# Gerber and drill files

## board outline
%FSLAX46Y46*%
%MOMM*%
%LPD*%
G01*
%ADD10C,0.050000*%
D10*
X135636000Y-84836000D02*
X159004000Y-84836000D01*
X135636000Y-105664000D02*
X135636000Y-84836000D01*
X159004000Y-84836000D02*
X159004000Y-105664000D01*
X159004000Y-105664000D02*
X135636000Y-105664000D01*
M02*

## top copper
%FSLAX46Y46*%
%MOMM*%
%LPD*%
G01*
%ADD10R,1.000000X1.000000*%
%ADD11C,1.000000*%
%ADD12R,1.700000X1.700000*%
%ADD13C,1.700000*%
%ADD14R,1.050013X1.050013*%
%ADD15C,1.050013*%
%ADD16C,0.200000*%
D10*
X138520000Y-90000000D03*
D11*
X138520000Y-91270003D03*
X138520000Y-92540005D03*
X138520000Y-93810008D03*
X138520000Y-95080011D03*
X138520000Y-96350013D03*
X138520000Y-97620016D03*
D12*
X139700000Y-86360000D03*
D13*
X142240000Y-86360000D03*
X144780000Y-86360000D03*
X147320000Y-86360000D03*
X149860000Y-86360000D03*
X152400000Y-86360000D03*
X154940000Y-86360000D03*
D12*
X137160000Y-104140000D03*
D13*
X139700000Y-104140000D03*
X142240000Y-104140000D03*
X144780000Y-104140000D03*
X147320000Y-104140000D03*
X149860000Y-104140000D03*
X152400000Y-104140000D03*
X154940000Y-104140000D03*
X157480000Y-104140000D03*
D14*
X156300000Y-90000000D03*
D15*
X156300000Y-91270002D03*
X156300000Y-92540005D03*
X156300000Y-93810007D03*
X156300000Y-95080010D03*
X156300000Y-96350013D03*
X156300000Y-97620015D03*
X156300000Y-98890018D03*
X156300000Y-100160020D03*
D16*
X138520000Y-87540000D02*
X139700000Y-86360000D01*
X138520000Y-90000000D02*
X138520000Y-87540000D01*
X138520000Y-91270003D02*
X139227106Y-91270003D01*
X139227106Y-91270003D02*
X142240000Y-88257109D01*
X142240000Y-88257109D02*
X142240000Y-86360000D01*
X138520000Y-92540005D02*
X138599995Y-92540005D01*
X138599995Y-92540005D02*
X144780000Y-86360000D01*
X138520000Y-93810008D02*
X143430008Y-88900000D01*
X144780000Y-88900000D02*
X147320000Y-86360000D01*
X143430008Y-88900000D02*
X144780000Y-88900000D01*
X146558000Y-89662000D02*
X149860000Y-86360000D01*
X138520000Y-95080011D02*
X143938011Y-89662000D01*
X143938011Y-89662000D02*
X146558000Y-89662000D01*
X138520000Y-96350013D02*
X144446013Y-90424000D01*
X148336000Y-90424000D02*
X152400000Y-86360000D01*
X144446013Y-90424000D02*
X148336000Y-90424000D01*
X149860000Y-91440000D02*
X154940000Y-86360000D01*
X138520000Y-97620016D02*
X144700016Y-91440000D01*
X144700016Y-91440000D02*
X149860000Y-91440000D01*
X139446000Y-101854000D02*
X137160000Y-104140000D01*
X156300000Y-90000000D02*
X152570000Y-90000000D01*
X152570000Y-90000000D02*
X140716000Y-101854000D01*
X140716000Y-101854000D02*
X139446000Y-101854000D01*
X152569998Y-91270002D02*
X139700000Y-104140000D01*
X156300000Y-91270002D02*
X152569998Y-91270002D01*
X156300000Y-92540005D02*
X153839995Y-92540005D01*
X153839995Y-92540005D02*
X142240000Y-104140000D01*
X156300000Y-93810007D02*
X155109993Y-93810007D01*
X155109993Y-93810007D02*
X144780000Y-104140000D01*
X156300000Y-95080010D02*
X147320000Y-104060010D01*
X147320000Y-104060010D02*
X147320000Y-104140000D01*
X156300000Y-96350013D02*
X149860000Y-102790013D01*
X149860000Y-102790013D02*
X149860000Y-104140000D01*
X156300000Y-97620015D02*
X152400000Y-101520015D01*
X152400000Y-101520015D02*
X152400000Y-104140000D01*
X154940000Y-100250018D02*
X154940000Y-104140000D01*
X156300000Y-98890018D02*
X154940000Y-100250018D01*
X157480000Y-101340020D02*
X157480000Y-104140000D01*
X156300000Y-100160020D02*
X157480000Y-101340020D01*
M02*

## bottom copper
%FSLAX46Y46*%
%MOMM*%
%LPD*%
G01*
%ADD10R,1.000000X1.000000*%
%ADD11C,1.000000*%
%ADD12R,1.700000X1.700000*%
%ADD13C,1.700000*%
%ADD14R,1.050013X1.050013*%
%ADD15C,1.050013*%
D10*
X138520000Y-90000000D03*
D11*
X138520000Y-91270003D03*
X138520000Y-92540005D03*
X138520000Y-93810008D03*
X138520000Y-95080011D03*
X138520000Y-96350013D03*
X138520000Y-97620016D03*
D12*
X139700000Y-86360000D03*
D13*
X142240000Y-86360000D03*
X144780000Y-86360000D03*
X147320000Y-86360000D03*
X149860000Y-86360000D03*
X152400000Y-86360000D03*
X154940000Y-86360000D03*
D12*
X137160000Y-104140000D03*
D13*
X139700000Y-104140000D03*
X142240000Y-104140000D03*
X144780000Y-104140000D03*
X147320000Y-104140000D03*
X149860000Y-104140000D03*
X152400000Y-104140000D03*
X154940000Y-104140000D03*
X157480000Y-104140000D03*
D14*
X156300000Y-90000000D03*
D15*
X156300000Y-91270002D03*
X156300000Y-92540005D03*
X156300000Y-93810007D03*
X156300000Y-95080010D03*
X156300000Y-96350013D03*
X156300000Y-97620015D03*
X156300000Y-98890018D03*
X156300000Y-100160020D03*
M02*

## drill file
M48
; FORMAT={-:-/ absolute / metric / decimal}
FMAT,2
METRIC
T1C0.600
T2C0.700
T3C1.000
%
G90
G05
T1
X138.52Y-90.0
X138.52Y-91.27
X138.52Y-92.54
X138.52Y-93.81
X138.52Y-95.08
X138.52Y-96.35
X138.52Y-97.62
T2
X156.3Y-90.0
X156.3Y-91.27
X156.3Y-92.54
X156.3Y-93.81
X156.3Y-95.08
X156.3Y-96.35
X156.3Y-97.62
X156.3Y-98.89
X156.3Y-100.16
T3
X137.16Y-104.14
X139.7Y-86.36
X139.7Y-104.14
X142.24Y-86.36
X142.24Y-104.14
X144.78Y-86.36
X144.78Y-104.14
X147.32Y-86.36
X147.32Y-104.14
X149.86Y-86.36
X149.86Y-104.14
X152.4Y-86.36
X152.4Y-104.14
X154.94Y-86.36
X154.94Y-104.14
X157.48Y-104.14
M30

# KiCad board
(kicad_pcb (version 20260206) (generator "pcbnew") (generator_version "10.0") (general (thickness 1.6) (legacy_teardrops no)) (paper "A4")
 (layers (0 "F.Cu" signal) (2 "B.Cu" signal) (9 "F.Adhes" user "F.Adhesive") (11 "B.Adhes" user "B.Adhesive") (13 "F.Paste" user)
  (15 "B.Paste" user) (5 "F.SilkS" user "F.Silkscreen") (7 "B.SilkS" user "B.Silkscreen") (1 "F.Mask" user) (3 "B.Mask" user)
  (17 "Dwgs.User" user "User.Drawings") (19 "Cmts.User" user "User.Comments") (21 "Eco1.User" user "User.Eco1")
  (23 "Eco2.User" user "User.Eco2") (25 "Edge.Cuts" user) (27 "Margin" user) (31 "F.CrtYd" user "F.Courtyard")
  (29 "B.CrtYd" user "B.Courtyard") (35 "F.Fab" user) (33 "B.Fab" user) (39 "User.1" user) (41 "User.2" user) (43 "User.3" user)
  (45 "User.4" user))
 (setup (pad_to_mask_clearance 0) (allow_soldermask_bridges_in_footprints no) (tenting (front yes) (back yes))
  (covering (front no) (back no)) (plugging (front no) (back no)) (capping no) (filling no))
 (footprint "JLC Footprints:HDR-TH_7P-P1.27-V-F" (layer "F.Cu") (at 138.52 93.810008 -90)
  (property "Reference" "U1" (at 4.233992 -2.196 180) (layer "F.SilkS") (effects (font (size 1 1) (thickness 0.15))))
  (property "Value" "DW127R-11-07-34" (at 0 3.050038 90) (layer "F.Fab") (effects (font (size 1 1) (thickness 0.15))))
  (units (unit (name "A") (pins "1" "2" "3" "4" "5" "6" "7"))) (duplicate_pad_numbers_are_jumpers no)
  (pad "1" thru_hole rect (at -3.810008 0 270) (size 1 1) (drill 0.6) (layers "*.Cu" "*.Mask") (remove_unused_layers no)
   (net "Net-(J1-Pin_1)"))
  (pad "2" thru_hole circle (at -2.540005 0 270) (size 1 1) (drill 0.6) (layers "*.Cu" "*.Mask") (remove_unused_layers no)
   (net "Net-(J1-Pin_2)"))
  (pad "3" thru_hole circle (at -1.270003 0 270) (size 1 1) (drill 0.6) (layers "*.Cu" "*.Mask") (remove_unused_layers no)
   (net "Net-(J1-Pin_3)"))
  (pad "4" thru_hole circle (at 0 0 270) (size 1 1) (drill 0.6) (layers "*.Cu" "*.Mask") (remove_unused_layers no) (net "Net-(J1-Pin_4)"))
  (pad "5" thru_hole circle (at 1.270003 0 270) (size 1 1) (drill 0.6) (layers "*.Cu" "*.Mask") (remove_unused_layers no)
   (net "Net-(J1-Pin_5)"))
  (pad "6" thru_hole circle (at 2.540005 0 270) (size 1 1) (drill 0.6) (layers "*.Cu" "*.Mask") (remove_unused_layers no)
   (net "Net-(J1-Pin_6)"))
  (pad "7" thru_hole circle (at 3.810008 0 270) (size 1 1) (drill 0.6) (layers "*.Cu" "*.Mask") (remove_unused_layers no)
   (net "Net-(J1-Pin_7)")))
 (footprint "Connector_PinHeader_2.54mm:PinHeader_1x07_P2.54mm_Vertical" (layer "F.Cu") (at 139.7 86.36 90)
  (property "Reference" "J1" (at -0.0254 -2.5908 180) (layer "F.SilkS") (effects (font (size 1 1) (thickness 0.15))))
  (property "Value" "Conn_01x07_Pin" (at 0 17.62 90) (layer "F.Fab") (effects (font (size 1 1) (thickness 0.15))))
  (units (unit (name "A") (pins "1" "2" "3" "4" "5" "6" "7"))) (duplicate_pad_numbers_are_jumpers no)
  (pad "1" thru_hole rect (at 0 0 90) (size 1.7 1.7) (drill 1) (layers "*.Cu" "*.Mask") (remove_unused_layers no) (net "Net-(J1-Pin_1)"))
  (pad "2" thru_hole circle (at 0 2.54 90) (size 1.7 1.7) (drill 1) (layers "*.Cu" "*.Mask") (remove_unused_layers no)
   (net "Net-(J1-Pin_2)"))
  (pad "3" thru_hole circle (at 0 5.08 90) (size 1.7 1.7) (drill 1) (layers "*.Cu" "*.Mask") (remove_unused_layers no)
   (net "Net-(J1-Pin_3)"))
  (pad "4" thru_hole circle (at 0 7.62 90) (size 1.7 1.7) (drill 1) (layers "*.Cu" "*.Mask") (remove_unused_layers no)
   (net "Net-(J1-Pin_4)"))
  (pad "5" thru_hole circle (at 0 10.16 90) (size 1.7 1.7) (drill 1) (layers "*.Cu" "*.Mask") (remove_unused_layers no)
   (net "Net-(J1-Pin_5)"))
  (pad "6" thru_hole circle (at 0 12.7 90) (size 1.7 1.7) (drill 1) (layers "*.Cu" "*.Mask") (remove_unused_layers no)
   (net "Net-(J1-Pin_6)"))
  (pad "7" thru_hole circle (at 0 15.24 90) (size 1.7 1.7) (drill 1) (layers "*.Cu" "*.Mask") (remove_unused_layers no)
   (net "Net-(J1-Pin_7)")))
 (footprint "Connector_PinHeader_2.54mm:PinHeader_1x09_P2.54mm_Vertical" (layer "F.Cu") (at 137.16 104.14 90)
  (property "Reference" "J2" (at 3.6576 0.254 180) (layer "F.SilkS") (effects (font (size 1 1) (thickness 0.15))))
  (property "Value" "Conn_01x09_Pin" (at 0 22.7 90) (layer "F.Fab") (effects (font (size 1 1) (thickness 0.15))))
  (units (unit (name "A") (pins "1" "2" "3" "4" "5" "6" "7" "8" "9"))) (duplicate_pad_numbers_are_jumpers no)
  (pad "1" thru_hole rect (at 0 0 90) (size 1.7 1.7) (drill 1) (layers "*.Cu" "*.Mask") (remove_unused_layers no) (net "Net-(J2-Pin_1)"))
  (pad "2" thru_hole circle (at 0 2.54 90) (size 1.7 1.7) (drill 1) (layers "*.Cu" "*.Mask") (remove_unused_layers no)
   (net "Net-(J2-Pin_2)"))
  (pad "3" thru_hole circle (at 0 5.08 90) (size 1.7 1.7) (drill 1) (layers "*.Cu" "*.Mask") (remove_unused_layers no)
   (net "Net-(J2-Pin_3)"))
  (pad "4" thru_hole circle (at 0 7.62 90) (size 1.7 1.7) (drill 1) (layers "*.Cu" "*.Mask") (remove_unused_layers no)
   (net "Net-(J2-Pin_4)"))
  (pad "5" thru_hole circle (at 0 10.16 90) (size 1.7 1.7) (drill 1) (layers "*.Cu" "*.Mask") (remove_unused_layers no)
   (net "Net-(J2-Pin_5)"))
  (pad "6" thru_hole circle (at 0 12.7 90) (size 1.7 1.7) (drill 1) (layers "*.Cu" "*.Mask") (remove_unused_layers no)
   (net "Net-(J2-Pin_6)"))
  (pad "7" thru_hole circle (at 0 15.24 90) (size 1.7 1.7) (drill 1) (layers "*.Cu" "*.Mask") (remove_unused_layers no)
   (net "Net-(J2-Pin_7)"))
  (pad "8" thru_hole circle (at 0 17.78 90) (size 1.7 1.7) (drill 1) (layers "*.Cu" "*.Mask") (remove_unused_layers no)
   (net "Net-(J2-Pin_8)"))
  (pad "9" thru_hole circle (at 0 20.32 90) (size 1.7 1.7) (drill 1) (layers "*.Cu" "*.Mask") (remove_unused_layers no)
   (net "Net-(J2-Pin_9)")))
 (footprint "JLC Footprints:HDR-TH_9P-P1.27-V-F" (layer "F.Cu") (at 156.3 95.08001 -90)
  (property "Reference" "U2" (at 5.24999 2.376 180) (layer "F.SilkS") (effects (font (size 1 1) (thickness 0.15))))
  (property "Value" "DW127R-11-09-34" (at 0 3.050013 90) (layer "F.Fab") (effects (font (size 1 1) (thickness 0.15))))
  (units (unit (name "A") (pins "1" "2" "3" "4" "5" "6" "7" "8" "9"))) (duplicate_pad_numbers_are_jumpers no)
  (pad "1" thru_hole rect (at -5.08001 0 270) (size 1.050013 1.050013) (drill 0.700025) (layers "*.Cu" "*.Mask") (remove_unused_layers no)
   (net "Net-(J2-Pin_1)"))
  (pad "2" thru_hole circle (at -3.810008 0 270) (size 1.050013 1.050013) (drill 0.700025) (layers "*.Cu" "*.Mask")
   (remove_unused_layers no) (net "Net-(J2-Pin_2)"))
  (pad "3" thru_hole circle (at -2.540005 0 270) (size 1.050013 1.050013) (drill 0.700025) (layers "*.Cu" "*.Mask")
   (remove_unused_layers no) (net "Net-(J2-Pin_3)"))
  (pad "4" thru_hole circle (at -1.270003 0 270) (size 1.050013 1.050013) (drill 0.700025) (layers "*.Cu" "*.Mask")
   (remove_unused_layers no) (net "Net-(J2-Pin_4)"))
  (pad "5" thru_hole circle (at 0 0 270) (size 1.050013 1.050013) (drill 0.700025) (layers "*.Cu" "*.Mask") (remove_unused_layers no)
   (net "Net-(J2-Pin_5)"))
  (pad "6" thru_hole circle (at 1.270003 0 270) (size 1.050013 1.050013) (drill 0.700025) (layers "*.Cu" "*.Mask") (remove_unused_layers no)
   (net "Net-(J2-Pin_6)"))
  (pad "7" thru_hole circle (at 2.540005 0 270) (size 1.050013 1.050013) (drill 0.700025) (layers "*.Cu" "*.Mask") (remove_unused_layers no)
   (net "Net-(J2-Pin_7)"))
  (pad "8" thru_hole circle (at 3.810008 0 270) (size 1.050013 1.050013) (drill 0.700025) (layers "*.Cu" "*.Mask") (remove_unused_layers no)
   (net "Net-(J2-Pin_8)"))
  (pad "9" thru_hole circle (at 5.08001 0 270) (size 1.050013 1.050013) (drill 0.700025) (layers "*.Cu" "*.Mask") (remove_unused_layers no)
   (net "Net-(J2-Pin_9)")))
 (gr_line (start 135.636 84.836) (end 159.004 84.836) (stroke (width 0.05) (type default)) (layer "Edge.Cuts"))
 (gr_line (start 135.636 105.664) (end 135.636 84.836) (stroke (width 0.05) (type default)) (layer "Edge.Cuts"))
 (gr_line (start 159.004 84.836) (end 159.004 105.664) (stroke (width 0.05) (type default)) (layer "Edge.Cuts"))
 (gr_line (start 159.004 105.664) (end 135.636 105.664) (stroke (width 0.05) (type default)) (layer "Edge.Cuts"))
 (segment (start 138.52 87.54) (end 139.7 86.36) (width 0.2) (layer "F.Cu") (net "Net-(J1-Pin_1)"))
 (segment (start 138.52 90) (end 138.52 87.54) (width 0.2) (layer "F.Cu") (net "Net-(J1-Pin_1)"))
 (segment (start 138.52 91.270003) (end 139.227106 91.270003) (width 0.2) (layer "F.Cu") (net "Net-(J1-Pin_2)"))
 (segment (start 139.227106 91.270003) (end 142.24 88.257109) (width 0.2) (layer "F.Cu") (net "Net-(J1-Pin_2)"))
 (segment (start 142.24 88.257109) (end 142.24 86.36) (width 0.2) (layer "F.Cu") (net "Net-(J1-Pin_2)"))
 (segment (start 138.52 92.540005) (end 138.599995 92.540005) (width 0.2) (layer "F.Cu") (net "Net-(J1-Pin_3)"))
 (segment (start 138.599995 92.540005) (end 144.78 86.36) (width 0.2) (layer "F.Cu") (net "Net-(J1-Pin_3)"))
 (segment (start 138.52 93.810008) (end 143.430008 88.9) (width 0.2) (layer "F.Cu") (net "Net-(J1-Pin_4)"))
 (segment (start 144.78 88.9) (end 147.32 86.36) (width 0.2) (layer "F.Cu") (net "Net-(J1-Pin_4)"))
 (segment (start 143.430008 88.9) (end 144.78 88.9) (width 0.2) (layer "F.Cu") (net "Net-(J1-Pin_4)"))
 (segment (start 146.558 89.662) (end 149.86 86.36) (width 0.2) (layer "F.Cu") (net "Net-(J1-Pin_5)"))
 (segment (start 138.52 95.080011) (end 143.938011 89.662) (width 0.2) (layer "F.Cu") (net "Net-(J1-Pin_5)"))
 (segment (start 143.938011 89.662) (end 146.558 89.662) (width 0.2) (layer "F.Cu") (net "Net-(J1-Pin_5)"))
 (segment (start 138.52 96.350013) (end 144.446013 90.424) (width 0.2) (layer "F.Cu") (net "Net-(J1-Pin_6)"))
 (segment (start 148.336 90.424) (end 152.4 86.36) (width 0.2) (layer "F.Cu") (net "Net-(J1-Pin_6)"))
 (segment (start 144.446013 90.424) (end 148.336 90.424) (width 0.2) (layer "F.Cu") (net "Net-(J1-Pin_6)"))
 (segment (start 149.86 91.44) (end 154.94 86.36) (width 0.2) (layer "F.Cu") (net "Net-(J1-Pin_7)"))
 (segment (start 138.52 97.620016) (end 144.700016 91.44) (width 0.2) (layer "F.Cu") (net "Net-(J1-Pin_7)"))
 (segment (start 144.700016 91.44) (end 149.86 91.44) (width 0.2) (layer "F.Cu") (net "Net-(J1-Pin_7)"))
 (segment (start 139.446 101.854) (end 137.16 104.14) (width 0.2) (layer "F.Cu") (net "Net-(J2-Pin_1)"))
 (segment (start 156.3 90) (end 152.57 90) (width 0.2) (layer "F.Cu") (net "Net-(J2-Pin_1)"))
 (segment (start 152.57 90) (end 140.716 101.854) (width 0.2) (layer "F.Cu") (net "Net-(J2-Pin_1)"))
 (segment (start 140.716 101.854) (end 139.446 101.854) (width 0.2) (layer "F.Cu") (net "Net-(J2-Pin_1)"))
 (segment (start 152.569998 91.270002) (end 139.7 104.14) (width 0.2) (layer "F.Cu") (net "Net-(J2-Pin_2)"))
 (segment (start 156.3 91.270002) (end 152.569998 91.270002) (width 0.2) (layer "F.Cu") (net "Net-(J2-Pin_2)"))
 (segment (start 156.3 92.540005) (end 153.839995 92.540005) (width 0.2) (layer "F.Cu") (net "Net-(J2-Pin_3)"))
 (segment (start 153.839995 92.540005) (end 142.24 104.14) (width 0.2) (layer "F.Cu") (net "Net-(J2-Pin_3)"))
 (segment (start 156.3 93.810007) (end 155.109993 93.810007) (width 0.2) (layer "F.Cu") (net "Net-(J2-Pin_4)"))
 (segment (start 155.109993 93.810007) (end 144.78 104.14) (width 0.2) (layer "F.Cu") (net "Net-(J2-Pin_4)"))
 (segment (start 156.3 95.08001) (end 147.32 104.06001) (width 0.2) (layer "F.Cu") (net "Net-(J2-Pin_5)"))
 (segment (start 147.32 104.06001) (end 147.32 104.14) (width 0.2) (layer "F.Cu") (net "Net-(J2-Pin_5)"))
 (segment (start 156.3 96.350013) (end 149.86 102.790013) (width 0.2) (layer "F.Cu") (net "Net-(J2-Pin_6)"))
 (segment (start 149.86 102.790013) (end 149.86 104.14) (width 0.2) (layer "F.Cu") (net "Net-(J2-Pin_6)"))
 (segment (start 156.3 97.620015) (end 152.4 101.520015) (width 0.2) (layer "F.Cu") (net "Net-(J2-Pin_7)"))
 (segment (start 152.4 101.520015) (end 152.4 104.14) (width 0.2) (layer "F.Cu") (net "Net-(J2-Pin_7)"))
 (segment (start 154.94 100.250018) (end 154.94 104.14) (width 0.2) (layer "F.Cu") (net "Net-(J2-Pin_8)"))
 (segment (start 156.3 98.890018) (end 154.94 100.250018) (width 0.2) (layer "F.Cu") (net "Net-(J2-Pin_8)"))
 (segment (start 157.48 101.34002) (end 157.48 104.14) (width 0.2) (layer "F.Cu") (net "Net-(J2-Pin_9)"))
 (segment (start 156.3 100.16002) (end 157.48 101.34002) (width 0.2) (layer "F.Cu") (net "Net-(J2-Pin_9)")))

